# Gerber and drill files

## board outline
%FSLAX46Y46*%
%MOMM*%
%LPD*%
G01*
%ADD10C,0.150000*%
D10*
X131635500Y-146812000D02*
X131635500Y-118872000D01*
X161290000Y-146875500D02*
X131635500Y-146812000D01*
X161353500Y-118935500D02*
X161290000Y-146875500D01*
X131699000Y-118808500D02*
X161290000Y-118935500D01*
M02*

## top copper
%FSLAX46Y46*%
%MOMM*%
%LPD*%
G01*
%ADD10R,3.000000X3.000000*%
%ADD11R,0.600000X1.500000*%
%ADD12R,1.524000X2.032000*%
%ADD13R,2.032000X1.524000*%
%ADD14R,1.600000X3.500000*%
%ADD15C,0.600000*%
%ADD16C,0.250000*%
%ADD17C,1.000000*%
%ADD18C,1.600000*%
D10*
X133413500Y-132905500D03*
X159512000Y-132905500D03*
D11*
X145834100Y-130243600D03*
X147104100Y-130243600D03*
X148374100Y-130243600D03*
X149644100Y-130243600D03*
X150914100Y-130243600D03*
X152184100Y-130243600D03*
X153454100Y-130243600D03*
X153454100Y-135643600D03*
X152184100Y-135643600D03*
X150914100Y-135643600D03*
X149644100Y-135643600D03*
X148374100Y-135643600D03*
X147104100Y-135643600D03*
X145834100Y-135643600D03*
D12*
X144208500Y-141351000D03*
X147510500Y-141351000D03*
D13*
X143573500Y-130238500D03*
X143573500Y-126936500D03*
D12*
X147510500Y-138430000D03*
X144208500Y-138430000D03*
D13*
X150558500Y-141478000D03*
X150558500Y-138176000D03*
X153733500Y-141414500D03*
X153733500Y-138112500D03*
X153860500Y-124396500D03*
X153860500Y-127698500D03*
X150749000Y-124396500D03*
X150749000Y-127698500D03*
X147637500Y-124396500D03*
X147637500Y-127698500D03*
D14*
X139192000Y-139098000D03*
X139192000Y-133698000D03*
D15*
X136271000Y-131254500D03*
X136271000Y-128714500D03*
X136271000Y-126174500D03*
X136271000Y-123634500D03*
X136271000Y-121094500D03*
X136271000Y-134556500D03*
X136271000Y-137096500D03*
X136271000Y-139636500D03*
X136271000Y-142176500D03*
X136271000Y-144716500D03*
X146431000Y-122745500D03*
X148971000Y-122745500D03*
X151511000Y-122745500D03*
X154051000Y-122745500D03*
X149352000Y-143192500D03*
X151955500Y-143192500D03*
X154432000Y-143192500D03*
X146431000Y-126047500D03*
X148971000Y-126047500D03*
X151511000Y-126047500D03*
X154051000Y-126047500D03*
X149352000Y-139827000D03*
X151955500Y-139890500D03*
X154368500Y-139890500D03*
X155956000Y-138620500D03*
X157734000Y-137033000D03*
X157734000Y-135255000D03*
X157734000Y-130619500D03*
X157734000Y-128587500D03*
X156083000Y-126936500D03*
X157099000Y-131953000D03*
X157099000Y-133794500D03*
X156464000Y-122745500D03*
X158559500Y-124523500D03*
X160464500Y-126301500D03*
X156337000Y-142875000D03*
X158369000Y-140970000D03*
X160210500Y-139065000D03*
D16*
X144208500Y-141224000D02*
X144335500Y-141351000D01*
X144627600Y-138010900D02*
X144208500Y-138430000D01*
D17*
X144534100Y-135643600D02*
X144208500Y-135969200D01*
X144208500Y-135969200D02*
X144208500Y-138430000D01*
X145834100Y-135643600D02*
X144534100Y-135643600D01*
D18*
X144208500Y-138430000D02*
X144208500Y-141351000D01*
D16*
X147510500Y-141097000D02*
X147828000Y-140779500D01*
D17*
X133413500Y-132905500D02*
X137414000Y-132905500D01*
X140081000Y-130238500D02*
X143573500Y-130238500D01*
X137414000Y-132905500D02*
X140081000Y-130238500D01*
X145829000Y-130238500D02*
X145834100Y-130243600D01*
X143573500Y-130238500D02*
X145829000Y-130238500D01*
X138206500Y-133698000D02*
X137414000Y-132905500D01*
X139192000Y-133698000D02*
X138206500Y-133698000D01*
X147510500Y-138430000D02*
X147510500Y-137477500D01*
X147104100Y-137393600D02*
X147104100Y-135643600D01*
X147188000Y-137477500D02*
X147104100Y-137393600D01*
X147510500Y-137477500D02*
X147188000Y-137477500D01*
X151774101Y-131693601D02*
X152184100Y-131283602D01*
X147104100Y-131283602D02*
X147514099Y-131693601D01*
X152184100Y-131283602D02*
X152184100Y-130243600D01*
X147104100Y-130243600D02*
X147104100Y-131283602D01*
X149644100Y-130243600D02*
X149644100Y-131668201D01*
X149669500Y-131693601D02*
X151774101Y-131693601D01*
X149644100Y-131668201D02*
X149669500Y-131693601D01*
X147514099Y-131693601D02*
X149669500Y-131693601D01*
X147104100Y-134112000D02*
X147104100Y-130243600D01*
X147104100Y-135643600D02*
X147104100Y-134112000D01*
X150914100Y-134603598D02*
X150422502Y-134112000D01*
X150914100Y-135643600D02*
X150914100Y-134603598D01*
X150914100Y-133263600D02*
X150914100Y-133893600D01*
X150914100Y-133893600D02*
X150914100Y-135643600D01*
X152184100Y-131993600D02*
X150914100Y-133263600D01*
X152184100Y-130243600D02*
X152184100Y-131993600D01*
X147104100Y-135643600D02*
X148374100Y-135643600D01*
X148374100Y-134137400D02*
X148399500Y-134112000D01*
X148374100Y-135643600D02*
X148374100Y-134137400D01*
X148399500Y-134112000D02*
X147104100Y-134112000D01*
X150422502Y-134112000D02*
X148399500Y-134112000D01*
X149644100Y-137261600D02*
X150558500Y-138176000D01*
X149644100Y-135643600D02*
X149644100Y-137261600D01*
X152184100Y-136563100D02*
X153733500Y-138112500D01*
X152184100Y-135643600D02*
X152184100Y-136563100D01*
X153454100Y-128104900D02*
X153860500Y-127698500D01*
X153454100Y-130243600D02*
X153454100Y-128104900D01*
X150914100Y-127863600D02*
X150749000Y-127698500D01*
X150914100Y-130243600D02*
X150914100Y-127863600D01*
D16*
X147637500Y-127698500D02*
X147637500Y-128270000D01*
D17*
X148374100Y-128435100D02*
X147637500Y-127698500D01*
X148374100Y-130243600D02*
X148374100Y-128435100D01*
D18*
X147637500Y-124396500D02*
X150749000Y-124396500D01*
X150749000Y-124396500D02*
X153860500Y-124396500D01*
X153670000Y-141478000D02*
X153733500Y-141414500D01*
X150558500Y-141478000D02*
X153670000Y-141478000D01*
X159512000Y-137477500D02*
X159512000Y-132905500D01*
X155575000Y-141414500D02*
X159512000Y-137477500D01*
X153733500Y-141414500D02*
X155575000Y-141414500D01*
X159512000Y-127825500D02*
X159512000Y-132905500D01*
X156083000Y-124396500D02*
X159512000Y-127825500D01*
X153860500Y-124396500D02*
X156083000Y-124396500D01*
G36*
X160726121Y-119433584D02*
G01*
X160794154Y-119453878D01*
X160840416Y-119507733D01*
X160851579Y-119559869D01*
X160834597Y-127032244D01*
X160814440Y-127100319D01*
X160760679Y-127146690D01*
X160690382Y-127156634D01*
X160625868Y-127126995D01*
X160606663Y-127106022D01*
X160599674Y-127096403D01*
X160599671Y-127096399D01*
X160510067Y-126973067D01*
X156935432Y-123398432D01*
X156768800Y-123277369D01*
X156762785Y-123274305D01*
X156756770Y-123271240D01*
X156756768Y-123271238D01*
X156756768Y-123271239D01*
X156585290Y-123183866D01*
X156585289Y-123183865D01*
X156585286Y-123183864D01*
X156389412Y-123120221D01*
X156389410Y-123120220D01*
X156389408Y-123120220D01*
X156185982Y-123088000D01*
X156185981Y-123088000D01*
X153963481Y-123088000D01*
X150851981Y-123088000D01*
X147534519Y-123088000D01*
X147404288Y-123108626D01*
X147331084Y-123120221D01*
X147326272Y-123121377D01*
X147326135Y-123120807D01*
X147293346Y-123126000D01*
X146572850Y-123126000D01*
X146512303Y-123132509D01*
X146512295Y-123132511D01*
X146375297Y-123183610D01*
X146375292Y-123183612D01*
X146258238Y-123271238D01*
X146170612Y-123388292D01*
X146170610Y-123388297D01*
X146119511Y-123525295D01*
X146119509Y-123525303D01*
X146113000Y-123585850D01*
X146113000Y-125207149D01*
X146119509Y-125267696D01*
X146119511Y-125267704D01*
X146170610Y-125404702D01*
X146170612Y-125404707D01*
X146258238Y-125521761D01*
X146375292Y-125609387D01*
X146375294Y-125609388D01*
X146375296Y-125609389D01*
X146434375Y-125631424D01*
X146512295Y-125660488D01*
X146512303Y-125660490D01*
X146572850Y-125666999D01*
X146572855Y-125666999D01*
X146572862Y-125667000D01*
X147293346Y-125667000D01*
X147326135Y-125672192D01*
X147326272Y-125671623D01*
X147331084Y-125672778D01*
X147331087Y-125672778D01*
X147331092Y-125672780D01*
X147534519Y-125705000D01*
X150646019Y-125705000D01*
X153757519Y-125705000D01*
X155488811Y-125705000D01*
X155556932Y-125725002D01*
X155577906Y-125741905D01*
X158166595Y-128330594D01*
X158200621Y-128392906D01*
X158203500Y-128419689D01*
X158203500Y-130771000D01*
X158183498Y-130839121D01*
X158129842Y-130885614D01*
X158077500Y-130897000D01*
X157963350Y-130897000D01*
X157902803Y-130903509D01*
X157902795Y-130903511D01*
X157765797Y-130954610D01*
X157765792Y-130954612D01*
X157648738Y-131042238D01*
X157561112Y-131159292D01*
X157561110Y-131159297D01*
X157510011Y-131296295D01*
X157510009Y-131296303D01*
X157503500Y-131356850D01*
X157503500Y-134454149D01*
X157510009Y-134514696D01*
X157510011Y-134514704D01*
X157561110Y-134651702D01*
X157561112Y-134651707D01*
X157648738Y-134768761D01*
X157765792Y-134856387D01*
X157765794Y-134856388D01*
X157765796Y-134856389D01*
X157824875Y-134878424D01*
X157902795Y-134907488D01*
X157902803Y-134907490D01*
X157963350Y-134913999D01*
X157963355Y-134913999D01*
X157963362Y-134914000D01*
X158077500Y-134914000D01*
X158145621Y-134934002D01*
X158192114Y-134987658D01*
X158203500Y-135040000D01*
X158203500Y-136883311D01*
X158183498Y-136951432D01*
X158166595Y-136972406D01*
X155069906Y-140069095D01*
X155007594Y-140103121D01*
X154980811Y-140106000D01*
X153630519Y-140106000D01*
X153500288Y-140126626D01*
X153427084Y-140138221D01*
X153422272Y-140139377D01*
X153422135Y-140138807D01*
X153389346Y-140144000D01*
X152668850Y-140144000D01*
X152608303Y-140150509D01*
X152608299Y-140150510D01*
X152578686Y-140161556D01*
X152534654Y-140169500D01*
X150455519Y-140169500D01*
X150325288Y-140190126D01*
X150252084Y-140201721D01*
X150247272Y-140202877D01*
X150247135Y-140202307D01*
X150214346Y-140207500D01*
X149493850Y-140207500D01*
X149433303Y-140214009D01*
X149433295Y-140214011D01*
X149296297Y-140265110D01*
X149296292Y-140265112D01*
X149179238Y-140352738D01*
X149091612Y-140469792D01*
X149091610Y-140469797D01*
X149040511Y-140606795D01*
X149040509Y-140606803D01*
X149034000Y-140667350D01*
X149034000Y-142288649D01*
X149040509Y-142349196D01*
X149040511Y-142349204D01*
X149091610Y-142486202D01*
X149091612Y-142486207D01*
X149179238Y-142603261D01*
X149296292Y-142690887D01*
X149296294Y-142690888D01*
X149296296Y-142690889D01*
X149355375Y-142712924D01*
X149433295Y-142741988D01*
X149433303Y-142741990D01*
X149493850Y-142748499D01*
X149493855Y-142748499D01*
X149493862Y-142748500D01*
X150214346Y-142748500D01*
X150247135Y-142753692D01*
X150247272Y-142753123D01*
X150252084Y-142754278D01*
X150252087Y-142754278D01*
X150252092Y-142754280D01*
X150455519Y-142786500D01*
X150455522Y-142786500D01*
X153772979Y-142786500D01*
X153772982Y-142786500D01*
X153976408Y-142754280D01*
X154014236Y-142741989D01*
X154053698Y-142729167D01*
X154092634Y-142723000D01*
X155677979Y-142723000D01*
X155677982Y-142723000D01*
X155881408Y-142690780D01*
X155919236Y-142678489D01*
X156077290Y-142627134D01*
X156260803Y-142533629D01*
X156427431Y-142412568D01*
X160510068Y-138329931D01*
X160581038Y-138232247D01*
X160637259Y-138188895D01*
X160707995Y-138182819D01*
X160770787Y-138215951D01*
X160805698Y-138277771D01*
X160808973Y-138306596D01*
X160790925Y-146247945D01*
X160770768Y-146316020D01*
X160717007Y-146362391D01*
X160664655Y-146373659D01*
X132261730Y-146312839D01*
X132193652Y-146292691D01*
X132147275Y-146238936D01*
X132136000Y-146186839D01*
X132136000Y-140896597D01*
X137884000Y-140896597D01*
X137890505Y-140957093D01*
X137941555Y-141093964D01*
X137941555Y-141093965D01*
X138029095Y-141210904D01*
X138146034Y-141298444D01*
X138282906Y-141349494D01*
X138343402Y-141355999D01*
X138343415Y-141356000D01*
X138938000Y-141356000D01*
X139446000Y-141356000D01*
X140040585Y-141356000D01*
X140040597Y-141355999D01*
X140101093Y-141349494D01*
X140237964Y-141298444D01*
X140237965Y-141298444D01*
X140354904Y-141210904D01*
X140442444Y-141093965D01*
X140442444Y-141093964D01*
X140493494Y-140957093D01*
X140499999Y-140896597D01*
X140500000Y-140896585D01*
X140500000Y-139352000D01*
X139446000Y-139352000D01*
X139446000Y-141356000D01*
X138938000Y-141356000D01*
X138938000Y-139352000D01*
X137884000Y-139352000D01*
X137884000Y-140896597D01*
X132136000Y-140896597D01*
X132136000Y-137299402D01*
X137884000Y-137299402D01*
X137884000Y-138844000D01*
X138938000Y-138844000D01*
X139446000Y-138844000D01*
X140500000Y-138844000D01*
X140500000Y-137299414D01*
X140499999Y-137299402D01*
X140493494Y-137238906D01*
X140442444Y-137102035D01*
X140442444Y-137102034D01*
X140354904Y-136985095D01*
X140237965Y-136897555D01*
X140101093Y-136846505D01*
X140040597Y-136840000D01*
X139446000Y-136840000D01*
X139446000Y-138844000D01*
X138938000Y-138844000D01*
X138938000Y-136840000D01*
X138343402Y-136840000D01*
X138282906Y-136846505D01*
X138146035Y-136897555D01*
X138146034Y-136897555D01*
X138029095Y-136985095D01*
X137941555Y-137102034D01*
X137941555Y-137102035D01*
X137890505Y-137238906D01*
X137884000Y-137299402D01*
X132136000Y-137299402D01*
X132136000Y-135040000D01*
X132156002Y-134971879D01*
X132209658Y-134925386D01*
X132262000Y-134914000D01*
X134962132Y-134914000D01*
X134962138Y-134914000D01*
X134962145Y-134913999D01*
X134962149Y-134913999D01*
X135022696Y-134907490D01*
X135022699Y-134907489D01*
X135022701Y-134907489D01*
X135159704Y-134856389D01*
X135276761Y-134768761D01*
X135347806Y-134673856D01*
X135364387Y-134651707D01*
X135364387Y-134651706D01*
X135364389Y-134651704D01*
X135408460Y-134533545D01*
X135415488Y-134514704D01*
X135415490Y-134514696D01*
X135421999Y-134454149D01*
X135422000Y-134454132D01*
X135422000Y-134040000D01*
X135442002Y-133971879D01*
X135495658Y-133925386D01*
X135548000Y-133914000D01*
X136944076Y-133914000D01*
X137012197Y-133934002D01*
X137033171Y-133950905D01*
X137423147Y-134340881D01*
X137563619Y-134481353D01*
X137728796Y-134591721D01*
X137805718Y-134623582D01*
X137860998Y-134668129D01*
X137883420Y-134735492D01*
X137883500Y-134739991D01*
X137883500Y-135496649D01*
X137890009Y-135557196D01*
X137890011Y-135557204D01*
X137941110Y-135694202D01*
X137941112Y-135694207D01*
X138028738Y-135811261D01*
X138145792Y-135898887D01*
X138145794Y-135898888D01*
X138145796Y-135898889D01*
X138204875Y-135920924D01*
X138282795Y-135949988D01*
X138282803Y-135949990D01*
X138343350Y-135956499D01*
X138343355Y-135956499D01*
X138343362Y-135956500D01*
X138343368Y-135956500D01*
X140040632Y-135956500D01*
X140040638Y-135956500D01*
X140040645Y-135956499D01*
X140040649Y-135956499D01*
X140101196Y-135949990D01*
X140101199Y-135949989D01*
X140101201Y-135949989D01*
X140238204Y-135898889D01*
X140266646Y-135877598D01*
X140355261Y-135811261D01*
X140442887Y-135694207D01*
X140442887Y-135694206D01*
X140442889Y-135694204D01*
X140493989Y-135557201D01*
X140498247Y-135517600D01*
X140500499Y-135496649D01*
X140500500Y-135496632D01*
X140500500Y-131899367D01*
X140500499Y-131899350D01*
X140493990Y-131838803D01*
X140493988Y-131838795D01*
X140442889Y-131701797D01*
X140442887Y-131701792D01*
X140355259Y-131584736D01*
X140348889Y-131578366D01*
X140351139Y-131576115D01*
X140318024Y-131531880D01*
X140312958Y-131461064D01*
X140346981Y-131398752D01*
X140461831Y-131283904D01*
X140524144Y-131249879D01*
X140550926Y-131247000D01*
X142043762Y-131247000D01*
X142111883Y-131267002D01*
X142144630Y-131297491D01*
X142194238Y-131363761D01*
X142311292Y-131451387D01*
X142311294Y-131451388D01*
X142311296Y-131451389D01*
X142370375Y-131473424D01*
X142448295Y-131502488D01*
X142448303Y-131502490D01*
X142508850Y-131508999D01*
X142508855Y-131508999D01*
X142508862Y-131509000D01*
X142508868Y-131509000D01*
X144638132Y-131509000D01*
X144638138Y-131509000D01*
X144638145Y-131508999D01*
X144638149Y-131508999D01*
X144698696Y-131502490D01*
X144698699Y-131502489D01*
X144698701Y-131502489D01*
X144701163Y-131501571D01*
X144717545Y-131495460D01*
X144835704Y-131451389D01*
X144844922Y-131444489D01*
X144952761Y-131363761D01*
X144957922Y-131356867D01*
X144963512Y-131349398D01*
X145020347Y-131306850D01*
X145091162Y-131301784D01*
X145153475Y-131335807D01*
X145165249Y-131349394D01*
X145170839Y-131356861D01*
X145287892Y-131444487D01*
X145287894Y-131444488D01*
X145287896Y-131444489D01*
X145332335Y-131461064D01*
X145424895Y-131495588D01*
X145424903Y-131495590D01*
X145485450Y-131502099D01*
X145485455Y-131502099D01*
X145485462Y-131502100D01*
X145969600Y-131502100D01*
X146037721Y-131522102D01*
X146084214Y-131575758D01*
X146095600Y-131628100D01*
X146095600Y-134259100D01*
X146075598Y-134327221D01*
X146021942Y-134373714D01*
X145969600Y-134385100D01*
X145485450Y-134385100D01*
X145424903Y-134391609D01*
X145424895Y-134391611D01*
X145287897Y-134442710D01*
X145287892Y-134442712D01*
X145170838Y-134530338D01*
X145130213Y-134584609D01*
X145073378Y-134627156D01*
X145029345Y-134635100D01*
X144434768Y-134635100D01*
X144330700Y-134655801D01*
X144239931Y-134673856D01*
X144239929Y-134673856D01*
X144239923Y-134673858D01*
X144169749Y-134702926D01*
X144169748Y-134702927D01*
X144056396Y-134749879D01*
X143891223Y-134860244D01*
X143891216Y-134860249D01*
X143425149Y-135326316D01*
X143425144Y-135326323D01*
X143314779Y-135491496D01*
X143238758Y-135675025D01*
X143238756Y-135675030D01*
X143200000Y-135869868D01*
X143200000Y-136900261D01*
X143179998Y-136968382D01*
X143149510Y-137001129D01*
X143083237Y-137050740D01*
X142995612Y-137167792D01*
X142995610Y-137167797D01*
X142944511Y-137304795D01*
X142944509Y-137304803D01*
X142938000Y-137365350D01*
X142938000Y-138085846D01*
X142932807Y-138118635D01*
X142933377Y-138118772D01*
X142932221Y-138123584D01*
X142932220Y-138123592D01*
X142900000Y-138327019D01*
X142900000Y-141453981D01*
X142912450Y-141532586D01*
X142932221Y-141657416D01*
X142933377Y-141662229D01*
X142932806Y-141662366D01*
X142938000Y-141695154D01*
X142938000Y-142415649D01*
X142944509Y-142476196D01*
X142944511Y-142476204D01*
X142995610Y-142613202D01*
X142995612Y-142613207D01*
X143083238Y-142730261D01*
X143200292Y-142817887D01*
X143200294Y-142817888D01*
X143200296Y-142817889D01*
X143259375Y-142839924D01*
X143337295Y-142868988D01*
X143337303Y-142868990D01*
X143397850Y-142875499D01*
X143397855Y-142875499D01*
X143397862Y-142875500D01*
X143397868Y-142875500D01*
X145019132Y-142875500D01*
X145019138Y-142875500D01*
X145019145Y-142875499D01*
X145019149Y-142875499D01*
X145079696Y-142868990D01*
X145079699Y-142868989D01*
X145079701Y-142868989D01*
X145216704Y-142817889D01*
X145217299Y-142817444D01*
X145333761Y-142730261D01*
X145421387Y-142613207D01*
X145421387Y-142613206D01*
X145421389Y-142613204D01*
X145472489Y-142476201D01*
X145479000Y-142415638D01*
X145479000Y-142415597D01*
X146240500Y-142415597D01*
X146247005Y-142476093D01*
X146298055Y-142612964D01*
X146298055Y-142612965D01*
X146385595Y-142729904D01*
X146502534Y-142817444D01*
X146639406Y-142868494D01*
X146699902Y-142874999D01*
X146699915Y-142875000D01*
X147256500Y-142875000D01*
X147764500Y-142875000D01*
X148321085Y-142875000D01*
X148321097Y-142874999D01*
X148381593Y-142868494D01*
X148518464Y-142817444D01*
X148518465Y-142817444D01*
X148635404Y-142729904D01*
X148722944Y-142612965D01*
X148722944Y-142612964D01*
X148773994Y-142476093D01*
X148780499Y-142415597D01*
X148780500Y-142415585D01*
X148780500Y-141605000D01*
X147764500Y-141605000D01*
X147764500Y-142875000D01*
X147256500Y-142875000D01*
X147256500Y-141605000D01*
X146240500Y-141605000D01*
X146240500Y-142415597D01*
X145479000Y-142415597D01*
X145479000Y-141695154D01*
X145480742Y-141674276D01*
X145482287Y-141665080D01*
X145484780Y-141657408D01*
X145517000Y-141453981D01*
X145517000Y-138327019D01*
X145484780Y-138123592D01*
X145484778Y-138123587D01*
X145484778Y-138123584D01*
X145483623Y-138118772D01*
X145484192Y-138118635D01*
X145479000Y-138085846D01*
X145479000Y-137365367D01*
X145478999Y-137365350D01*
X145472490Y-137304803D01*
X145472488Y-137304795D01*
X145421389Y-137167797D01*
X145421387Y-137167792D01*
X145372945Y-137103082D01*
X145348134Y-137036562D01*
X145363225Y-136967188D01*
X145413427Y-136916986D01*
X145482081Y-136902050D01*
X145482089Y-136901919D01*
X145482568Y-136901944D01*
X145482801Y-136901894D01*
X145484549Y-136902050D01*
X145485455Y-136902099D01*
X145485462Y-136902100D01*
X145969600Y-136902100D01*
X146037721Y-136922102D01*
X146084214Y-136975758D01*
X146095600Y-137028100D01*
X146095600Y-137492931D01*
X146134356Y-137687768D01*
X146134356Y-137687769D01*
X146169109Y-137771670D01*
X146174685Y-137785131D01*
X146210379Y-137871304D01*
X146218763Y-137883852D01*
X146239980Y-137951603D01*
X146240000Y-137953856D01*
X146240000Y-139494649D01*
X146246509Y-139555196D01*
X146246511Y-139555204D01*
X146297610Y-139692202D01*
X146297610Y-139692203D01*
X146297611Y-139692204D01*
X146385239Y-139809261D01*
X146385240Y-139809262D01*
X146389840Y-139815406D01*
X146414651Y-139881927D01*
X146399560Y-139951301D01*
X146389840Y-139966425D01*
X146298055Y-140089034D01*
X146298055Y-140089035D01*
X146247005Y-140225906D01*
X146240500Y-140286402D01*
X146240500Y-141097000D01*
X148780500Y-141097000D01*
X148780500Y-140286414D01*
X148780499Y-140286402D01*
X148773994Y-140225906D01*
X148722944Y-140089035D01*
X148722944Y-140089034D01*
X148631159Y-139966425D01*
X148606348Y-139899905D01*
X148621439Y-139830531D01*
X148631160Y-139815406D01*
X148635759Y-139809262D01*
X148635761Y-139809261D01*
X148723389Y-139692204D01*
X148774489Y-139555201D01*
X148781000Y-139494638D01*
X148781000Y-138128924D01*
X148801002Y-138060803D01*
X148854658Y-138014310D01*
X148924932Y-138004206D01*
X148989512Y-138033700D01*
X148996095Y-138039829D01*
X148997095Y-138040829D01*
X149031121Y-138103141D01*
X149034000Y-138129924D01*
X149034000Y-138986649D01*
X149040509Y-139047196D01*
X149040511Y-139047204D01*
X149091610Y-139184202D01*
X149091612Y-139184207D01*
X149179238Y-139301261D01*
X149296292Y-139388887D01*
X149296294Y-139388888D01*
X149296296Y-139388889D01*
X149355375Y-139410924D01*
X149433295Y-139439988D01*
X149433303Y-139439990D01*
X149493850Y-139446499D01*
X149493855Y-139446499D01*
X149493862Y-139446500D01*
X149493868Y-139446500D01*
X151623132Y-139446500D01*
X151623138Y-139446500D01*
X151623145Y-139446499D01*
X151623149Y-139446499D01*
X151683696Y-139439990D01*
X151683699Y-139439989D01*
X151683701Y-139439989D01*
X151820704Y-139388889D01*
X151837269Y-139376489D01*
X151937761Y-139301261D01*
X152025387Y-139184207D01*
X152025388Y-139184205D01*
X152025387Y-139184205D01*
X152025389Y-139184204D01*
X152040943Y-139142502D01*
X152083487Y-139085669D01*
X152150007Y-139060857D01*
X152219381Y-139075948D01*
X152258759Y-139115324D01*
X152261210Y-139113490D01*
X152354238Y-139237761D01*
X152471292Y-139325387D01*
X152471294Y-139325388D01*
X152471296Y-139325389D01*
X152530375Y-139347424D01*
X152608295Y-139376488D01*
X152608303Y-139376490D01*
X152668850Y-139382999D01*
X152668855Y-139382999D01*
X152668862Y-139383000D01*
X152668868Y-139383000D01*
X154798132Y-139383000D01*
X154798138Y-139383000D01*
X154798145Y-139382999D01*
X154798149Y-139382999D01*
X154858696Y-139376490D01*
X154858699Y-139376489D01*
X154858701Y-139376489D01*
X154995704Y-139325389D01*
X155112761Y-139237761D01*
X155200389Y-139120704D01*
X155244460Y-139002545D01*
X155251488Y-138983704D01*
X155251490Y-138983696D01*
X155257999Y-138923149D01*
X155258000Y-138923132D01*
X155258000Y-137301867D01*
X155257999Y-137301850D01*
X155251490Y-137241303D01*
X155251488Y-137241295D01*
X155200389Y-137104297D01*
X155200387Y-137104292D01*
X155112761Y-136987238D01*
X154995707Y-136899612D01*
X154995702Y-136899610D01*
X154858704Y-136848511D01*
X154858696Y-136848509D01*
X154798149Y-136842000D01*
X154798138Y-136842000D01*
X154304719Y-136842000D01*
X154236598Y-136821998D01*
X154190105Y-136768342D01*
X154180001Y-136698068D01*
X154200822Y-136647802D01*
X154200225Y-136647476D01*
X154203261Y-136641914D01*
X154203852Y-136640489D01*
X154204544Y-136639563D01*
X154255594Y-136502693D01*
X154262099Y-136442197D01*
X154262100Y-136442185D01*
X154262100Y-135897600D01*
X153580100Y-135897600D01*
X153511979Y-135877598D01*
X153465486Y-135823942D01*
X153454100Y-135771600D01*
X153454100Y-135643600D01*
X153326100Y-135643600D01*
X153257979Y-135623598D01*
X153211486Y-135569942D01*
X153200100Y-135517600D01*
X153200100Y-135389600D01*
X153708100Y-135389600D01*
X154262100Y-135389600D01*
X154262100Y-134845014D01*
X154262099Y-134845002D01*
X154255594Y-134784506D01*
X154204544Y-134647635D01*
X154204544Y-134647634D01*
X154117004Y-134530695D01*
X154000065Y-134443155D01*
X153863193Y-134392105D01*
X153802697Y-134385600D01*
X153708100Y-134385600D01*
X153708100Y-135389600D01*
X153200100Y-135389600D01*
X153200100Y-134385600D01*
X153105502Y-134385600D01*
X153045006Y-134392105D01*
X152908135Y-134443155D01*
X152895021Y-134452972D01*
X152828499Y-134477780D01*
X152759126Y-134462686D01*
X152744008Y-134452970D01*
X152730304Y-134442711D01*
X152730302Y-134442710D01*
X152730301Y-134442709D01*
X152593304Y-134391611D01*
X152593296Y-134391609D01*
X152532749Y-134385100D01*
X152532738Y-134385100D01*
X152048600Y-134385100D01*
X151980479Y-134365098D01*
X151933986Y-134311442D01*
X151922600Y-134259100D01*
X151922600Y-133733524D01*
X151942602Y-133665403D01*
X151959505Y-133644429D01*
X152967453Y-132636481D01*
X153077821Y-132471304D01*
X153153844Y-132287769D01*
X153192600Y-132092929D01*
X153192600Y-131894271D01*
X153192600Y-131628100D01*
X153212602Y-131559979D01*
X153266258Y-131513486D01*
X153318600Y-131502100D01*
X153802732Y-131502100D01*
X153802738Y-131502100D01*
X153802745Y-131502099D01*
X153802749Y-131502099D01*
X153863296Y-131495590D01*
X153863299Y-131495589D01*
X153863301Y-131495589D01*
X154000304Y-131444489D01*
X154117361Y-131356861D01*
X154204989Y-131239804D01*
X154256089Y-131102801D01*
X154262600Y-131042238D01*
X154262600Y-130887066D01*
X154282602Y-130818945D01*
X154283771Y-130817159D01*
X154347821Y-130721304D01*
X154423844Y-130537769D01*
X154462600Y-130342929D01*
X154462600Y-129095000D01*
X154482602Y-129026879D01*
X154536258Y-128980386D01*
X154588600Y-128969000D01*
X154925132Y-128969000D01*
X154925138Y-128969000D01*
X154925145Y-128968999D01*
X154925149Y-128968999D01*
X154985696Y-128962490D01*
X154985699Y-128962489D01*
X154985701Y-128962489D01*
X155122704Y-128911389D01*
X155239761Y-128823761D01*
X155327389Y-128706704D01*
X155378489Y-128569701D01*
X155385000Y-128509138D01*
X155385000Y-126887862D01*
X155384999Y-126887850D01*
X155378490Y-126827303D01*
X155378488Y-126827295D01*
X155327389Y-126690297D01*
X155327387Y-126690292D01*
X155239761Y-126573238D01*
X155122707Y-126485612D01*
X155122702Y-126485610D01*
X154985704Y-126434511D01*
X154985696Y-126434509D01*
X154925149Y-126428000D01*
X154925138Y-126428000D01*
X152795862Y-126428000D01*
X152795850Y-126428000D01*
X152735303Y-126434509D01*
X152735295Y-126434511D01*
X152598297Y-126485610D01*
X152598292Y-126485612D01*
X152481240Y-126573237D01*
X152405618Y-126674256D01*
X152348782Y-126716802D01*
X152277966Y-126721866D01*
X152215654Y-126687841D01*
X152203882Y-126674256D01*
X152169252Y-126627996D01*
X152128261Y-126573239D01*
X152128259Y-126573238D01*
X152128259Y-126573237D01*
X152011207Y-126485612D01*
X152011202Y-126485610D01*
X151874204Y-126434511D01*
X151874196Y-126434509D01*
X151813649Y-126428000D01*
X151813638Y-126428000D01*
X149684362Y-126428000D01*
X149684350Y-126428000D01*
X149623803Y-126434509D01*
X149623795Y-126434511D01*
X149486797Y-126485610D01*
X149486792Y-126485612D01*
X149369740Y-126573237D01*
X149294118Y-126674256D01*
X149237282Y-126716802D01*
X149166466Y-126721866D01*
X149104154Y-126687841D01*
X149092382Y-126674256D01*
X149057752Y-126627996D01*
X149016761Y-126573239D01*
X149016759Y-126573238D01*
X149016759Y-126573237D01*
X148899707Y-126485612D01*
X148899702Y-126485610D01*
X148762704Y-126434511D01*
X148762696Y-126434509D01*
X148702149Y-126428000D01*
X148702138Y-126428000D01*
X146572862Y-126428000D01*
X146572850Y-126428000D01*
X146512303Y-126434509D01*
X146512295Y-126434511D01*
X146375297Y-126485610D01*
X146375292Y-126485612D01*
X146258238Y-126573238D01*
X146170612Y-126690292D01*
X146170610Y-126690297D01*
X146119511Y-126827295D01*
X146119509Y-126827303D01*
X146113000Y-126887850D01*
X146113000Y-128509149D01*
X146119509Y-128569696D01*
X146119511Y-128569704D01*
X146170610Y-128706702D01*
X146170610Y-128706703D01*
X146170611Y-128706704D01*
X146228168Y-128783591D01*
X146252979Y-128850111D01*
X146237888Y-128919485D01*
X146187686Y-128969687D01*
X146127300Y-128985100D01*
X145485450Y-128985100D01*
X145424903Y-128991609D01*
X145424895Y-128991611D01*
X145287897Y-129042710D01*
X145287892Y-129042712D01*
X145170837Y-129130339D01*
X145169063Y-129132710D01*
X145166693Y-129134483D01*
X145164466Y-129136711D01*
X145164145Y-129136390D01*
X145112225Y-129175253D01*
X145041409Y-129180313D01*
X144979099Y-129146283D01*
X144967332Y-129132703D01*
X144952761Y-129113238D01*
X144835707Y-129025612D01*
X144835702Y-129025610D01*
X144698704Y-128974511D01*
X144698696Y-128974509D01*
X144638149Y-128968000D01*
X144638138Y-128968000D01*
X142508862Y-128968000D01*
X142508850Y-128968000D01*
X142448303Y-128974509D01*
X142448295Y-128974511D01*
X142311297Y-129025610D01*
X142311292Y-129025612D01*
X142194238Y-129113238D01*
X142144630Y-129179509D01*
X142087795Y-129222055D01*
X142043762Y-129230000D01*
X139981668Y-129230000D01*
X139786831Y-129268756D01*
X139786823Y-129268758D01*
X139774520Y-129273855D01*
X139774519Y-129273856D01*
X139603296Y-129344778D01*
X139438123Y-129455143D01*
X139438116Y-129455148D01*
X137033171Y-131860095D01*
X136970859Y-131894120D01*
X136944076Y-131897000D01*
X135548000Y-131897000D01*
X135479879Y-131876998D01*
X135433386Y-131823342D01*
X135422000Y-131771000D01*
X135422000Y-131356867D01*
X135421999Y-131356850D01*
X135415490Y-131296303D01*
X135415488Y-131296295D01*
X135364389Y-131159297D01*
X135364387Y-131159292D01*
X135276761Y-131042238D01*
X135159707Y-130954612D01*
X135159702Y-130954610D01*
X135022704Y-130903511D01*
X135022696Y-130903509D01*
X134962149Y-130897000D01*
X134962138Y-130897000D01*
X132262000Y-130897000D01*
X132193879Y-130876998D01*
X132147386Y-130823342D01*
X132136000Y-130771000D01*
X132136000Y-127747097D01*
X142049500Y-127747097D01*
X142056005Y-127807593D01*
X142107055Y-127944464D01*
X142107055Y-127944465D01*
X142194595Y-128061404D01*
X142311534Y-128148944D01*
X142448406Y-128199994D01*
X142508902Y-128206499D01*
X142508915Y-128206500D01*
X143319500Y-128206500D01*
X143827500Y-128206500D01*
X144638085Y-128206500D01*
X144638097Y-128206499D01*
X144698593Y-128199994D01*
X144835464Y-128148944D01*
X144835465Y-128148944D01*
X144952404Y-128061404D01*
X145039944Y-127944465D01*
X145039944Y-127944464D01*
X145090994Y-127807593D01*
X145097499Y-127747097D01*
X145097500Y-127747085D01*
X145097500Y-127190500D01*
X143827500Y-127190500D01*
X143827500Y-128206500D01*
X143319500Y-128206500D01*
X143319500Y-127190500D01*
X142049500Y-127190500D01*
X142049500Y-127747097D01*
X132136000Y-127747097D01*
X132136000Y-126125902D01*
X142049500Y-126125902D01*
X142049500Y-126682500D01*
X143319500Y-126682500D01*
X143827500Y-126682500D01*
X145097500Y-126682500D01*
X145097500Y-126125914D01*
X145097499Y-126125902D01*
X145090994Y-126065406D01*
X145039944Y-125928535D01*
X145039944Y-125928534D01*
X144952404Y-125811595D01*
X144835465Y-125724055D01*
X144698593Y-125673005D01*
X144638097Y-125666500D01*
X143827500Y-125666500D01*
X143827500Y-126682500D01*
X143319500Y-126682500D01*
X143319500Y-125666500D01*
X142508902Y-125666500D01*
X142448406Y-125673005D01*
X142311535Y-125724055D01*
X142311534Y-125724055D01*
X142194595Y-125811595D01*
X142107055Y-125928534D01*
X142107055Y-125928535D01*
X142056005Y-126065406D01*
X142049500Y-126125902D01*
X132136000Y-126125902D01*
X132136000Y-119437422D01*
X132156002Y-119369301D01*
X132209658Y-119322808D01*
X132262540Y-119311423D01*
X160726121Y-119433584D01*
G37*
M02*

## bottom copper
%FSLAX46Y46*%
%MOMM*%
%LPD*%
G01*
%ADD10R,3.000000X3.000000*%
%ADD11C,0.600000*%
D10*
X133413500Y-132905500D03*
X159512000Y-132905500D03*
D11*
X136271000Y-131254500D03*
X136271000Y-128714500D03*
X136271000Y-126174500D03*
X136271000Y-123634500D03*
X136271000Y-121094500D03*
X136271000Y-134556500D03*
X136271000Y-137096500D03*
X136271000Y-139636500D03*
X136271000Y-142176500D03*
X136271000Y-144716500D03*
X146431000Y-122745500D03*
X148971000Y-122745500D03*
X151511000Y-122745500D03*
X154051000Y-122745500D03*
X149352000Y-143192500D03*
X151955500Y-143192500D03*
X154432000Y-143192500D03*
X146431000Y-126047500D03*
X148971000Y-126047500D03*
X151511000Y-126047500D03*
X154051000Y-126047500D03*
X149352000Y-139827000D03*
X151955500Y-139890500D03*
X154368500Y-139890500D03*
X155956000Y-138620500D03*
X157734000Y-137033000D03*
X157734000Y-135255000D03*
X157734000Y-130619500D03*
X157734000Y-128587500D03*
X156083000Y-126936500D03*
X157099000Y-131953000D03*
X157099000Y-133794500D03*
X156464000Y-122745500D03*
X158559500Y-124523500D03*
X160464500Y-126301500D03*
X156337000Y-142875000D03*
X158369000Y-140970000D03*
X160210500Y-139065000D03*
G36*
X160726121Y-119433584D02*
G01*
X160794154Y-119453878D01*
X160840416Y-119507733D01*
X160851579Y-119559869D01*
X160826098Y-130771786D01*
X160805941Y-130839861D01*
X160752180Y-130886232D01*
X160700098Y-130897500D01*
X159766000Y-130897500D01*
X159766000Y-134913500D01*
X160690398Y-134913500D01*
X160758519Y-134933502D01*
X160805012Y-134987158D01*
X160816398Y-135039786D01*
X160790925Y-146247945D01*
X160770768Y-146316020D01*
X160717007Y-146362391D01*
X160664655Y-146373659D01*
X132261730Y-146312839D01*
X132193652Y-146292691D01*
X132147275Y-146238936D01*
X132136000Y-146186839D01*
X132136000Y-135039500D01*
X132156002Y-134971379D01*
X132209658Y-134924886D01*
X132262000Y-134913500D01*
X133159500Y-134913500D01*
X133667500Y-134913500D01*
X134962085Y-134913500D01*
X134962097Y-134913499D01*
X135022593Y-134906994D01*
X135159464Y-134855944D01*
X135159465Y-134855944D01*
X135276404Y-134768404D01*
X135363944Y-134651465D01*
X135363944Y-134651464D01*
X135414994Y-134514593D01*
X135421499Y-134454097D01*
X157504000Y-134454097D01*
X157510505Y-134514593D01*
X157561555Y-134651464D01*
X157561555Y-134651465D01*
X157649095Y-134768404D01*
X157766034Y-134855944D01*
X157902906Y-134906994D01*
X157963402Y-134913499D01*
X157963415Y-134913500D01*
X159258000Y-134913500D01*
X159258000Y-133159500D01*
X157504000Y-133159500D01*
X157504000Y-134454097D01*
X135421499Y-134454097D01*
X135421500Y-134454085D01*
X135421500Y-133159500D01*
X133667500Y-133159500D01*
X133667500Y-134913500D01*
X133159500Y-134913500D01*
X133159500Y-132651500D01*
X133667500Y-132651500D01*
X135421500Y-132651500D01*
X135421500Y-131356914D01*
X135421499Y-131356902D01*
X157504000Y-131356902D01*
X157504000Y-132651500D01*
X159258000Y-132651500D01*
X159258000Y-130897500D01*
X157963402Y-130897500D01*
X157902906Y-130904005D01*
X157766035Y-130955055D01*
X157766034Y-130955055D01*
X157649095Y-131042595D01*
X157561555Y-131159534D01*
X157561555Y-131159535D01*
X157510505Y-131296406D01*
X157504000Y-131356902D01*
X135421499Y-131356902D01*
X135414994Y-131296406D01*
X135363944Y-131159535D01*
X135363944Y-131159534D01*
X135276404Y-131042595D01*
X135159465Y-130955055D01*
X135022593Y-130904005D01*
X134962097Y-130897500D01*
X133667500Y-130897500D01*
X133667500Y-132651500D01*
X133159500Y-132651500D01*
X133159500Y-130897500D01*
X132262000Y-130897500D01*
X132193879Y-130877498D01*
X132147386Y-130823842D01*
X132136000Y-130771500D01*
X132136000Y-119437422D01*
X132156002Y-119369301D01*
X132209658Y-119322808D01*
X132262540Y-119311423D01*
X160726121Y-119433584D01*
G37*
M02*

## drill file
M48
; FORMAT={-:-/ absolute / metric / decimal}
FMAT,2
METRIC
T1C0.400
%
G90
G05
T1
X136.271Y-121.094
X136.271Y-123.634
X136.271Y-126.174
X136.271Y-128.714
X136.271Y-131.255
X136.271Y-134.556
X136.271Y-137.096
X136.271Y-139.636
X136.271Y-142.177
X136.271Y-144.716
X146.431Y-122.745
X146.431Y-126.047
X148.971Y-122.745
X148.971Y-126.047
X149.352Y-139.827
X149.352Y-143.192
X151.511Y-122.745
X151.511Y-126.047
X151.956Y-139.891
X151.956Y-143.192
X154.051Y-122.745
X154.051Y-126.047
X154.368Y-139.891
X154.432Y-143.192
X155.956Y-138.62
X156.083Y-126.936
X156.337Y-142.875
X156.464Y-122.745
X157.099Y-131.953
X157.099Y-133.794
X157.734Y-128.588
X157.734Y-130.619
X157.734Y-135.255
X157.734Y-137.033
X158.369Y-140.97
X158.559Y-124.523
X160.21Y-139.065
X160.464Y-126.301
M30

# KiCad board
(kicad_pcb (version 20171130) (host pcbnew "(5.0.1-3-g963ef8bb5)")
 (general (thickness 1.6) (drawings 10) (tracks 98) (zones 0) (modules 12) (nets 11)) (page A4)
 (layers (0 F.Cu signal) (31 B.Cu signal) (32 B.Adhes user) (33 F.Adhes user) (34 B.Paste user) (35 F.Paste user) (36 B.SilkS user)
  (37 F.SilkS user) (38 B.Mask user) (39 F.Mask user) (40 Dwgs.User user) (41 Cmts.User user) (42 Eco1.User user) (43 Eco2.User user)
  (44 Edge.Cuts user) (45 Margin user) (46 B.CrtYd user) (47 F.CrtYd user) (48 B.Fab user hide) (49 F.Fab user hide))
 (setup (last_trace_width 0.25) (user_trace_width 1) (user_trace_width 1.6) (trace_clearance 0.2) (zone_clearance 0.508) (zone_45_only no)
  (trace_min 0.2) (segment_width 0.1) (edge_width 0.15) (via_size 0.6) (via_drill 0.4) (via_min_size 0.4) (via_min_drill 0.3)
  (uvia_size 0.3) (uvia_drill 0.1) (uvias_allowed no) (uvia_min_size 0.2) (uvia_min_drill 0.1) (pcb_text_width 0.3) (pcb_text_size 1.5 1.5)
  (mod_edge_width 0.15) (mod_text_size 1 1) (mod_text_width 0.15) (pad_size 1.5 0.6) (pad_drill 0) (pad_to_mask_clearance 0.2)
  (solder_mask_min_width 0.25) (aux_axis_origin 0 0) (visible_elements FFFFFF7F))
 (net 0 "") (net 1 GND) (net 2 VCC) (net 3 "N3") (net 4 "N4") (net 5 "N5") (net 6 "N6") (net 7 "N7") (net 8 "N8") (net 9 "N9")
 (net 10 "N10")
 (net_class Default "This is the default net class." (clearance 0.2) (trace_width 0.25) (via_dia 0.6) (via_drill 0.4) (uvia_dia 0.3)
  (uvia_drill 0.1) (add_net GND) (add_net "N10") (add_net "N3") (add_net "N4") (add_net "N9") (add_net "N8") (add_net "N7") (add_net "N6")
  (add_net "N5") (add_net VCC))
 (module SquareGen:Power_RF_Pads (layer F.Cu) (at 133.4135 132.9055)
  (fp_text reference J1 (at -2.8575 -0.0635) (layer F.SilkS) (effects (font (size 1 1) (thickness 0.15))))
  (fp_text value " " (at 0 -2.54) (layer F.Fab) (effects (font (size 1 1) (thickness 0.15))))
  (pad 2 smd rect (at 0 0) (size 3 3) (layers B.Cu B.Paste B.Mask) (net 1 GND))
  (pad 1 smd rect (at 0 0) (size 3 3) (layers F.Cu F.Paste F.Mask) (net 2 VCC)))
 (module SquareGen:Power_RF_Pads (layer F.Cu) (at 159.512 132.9055)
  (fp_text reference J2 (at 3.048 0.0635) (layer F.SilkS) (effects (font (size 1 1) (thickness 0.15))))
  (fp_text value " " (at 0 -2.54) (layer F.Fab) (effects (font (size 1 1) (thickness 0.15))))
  (pad 2 smd rect (at 0 0) (size 3 3) (layers B.Cu B.Paste B.Mask) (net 1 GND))
  (pad 1 smd rect (at 0 0) (size 3 3) (layers F.Cu F.Paste F.Mask) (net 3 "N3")))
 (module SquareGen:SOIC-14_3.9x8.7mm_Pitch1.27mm (layer F.Cu) (at 149.6441 132.9436 90)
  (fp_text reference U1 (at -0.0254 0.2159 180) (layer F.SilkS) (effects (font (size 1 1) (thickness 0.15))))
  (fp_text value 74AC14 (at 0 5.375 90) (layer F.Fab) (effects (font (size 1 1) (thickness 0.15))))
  (pad 14 smd rect (at 2.7 -3.81 90) (size 1.5 0.6) (layers F.Cu F.Paste F.Mask) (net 2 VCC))
  (pad 13 smd rect (at 2.7 -2.54 90) (size 1.5 0.6) (layers F.Cu F.Paste F.Mask) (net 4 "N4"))
  (pad 12 smd rect (at 2.7 -1.27 90) (size 1.5 0.6) (layers F.Cu F.Paste F.Mask) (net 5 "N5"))
  (pad 11 smd rect (at 2.7 0 90) (size 1.5 0.6) (layers F.Cu F.Paste F.Mask) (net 4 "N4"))
  (pad 10 smd rect (at 2.7 1.27 90) (size 1.5 0.6) (layers F.Cu F.Paste F.Mask) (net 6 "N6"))
  (pad 9 smd rect (at 2.7 2.54 90) (size 1.5 0.6) (layers F.Cu F.Paste F.Mask) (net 4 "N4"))
  (pad 8 smd rect (at 2.7 3.81 90) (size 1.5 0.6) (layers F.Cu F.Paste F.Mask) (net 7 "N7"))
  (pad 7 smd rect (at -2.7 3.81 90) (size 1.5 0.6) (layers F.Cu F.Paste F.Mask) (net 1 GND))
  (pad 6 smd rect (at -2.7 2.54 90) (size 1.5 0.6) (layers F.Cu F.Paste F.Mask) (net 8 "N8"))
  (pad 5 smd rect (at -2.7 1.27 90) (size 1.5 0.6) (layers F.Cu F.Paste F.Mask) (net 4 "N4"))
  (pad 4 smd rect (at -2.7 0 90) (size 1.5 0.6) (layers F.Cu F.Paste F.Mask) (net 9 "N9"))
  (pad 3 smd rect (at -2.7 -1.27 90) (size 1.5 0.6) (layers F.Cu F.Paste F.Mask) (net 4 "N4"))
  (pad 2 smd rect (at -2.7 -2.54 90) (size 1.5 0.6) (layers F.Cu F.Paste F.Mask) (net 4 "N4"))
  (pad 1 smd rect (at -2.7 -3.81 90) (size 1.5 0.6) (layers F.Cu F.Paste F.Mask) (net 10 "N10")))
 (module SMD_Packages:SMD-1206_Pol (layer F.Cu) (at 145.8595 141.351)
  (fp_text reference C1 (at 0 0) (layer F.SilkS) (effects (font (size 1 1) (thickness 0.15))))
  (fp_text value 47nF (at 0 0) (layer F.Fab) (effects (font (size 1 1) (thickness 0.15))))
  (pad 1 smd rect (at -1.651 0) (size 1.524 2.032) (layers F.Cu F.Paste F.Mask) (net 10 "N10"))
  (pad 2 smd rect (at 1.651 0) (size 1.524 2.032) (layers F.Cu F.Paste F.Mask) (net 1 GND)))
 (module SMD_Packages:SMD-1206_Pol (layer F.Cu) (at 143.5735 128.5875 90)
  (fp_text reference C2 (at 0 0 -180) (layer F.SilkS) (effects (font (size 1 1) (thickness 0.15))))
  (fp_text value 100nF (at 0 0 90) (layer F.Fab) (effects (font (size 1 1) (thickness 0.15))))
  (pad 1 smd rect (at -1.651 0 90) (size 1.524 2.032) (layers F.Cu F.Paste F.Mask) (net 2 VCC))
  (pad 2 smd rect (at 1.651 0 90) (size 1.524 2.032) (layers F.Cu F.Paste F.Mask) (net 1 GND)))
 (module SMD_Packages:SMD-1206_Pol (layer F.Cu) (at 145.8595 138.43 180)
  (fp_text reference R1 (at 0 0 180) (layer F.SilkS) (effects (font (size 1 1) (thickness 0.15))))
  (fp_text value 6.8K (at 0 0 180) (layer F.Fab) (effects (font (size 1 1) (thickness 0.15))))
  (pad 1 smd rect (at -1.651 0 180) (size 1.524 2.032) (layers F.Cu F.Paste F.Mask) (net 4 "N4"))
  (pad 2 smd rect (at 1.651 0 180) (size 1.524 2.032) (layers F.Cu F.Paste F.Mask) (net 10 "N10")))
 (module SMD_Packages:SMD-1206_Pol (layer F.Cu) (at 150.5585 139.827 90)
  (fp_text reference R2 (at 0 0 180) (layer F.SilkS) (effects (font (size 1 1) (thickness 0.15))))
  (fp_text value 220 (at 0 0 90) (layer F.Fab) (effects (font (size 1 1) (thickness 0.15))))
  (pad 1 smd rect (at -1.651 0 90) (size 1.524 2.032) (layers F.Cu F.Paste F.Mask) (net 3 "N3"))
  (pad 2 smd rect (at 1.651 0 90) (size 1.524 2.032) (layers F.Cu F.Paste F.Mask) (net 9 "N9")))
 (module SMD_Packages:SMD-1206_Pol (layer F.Cu) (at 153.7335 139.7635 90)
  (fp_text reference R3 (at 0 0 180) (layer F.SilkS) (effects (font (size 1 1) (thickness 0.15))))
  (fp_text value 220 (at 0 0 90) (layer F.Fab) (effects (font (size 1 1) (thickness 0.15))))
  (pad 1 smd rect (at -1.651 0 90) (size 1.524 2.032) (layers F.Cu F.Paste F.Mask) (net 3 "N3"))
  (pad 2 smd rect (at 1.651 0 90) (size 1.524 2.032) (layers F.Cu F.Paste F.Mask) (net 8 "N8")))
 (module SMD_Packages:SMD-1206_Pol (layer F.Cu) (at 153.8605 126.0475 270)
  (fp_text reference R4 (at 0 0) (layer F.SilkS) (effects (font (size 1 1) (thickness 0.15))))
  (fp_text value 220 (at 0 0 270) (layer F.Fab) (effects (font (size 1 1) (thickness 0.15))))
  (pad 1 smd rect (at -1.651 0 270) (size 1.524 2.032) (layers F.Cu F.Paste F.Mask) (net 3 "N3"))
  (pad 2 smd rect (at 1.651 0 270) (size 1.524 2.032) (layers F.Cu F.Paste F.Mask) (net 7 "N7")))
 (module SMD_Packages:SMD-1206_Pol (layer F.Cu) (at 150.749 126.0475 270)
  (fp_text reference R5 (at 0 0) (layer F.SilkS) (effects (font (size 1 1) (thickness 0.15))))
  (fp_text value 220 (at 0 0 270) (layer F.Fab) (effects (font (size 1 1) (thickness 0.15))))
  (pad 1 smd rect (at -1.651 0 270) (size 1.524 2.032) (layers F.Cu F.Paste F.Mask) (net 3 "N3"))
  (pad 2 smd rect (at 1.651 0 270) (size 1.524 2.032) (layers F.Cu F.Paste F.Mask) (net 6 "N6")))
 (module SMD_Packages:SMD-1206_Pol (layer F.Cu) (at 147.6375 126.0475 270)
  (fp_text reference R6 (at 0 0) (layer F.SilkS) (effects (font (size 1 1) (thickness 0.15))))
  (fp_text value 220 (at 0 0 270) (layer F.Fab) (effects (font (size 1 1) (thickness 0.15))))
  (pad 1 smd rect (at -1.651 0 270) (size 1.524 2.032) (layers F.Cu F.Paste F.Mask) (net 3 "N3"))
  (pad 2 smd rect (at 1.651 0 270) (size 1.524 2.032) (layers F.Cu F.Paste F.Mask) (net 5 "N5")))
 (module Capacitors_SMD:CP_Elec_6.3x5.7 (layer F.Cu) (at 139.192 136.398 270)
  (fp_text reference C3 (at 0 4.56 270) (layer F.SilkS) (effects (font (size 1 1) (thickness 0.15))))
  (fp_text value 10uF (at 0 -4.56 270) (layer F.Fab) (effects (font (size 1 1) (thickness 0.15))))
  (pad 2 smd rect (at 2.7 0 90) (size 3.5 1.6) (layers F.Cu F.Paste F.Mask) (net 1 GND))
  (pad 1 smd rect (at -2.7 0 90) (size 3.5 1.6) (layers F.Cu F.Paste F.Mask) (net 2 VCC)))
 (gr_line (start 131.6355 146.812) (end 131.6355 118.872) (angle 90) (layer Edge.Cuts) (width 0.15))
 (gr_line (start 161.29 146.8755) (end 131.6355 146.812) (angle 90) (layer Edge.Cuts) (width 0.15))
 (gr_line (start 161.3535 118.9355) (end 161.29 146.8755) (angle 90) (layer Edge.Cuts) (width 0.15))
 (gr_line (start 131.699 118.8085) (end 161.29 118.9355) (angle 90) (layer Edge.Cuts) (width 0.15))
 (segment (start 144.2085 141.224) (end 144.3355 141.351) (width 0.25) (layer F.Cu) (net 10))
 (segment (start 144.6276 138.0109) (end 144.2085 138.43) (width 0.25) (layer F.Cu) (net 10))
 (segment (start 144.5341 135.6436) (end 144.2085 135.9692) (width 1) (layer F.Cu) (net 10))
 (segment (start 144.2085 135.9692) (end 144.2085 138.43) (width 1) (layer F.Cu) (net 10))
 (segment (start 145.8341 135.6436) (end 144.5341 135.6436) (width 1) (layer F.Cu) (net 10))
 (segment (start 144.2085 138.43) (end 144.2085 141.351) (width 1.6) (layer F.Cu) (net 10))
 (via (at 136.271 131.2545) (size 0.6) (drill 0.4) (layers F.Cu B.Cu) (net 1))
 (via (at 136.271 128.7145) (size 0.6) (drill 0.4) (layers F.Cu B.Cu) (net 1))
 (via (at 136.271 126.1745) (size 0.6) (drill 0.4) (layers F.Cu B.Cu) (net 1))
 (via (at 136.271 123.6345) (size 0.6) (drill 0.4) (layers F.Cu B.Cu) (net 1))
 (via (at 136.271 121.0945) (size 0.6) (drill 0.4) (layers F.Cu B.Cu) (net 1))
 (via (at 136.271 134.5565) (size 0.6) (drill 0.4) (layers F.Cu B.Cu) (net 1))
 (via (at 136.271 137.0965) (size 0.6) (drill 0.4) (layers F.Cu B.Cu) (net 1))
 (via (at 136.271 139.6365) (size 0.6) (drill 0.4) (layers F.Cu B.Cu) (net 1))
 (via (at 136.271 142.1765) (size 0.6) (drill 0.4) (layers F.Cu B.Cu) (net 1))
 (via (at 136.271 144.7165) (size 0.6) (drill 0.4) (layers F.Cu B.Cu) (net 1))
 (via (at 146.431 122.7455) (size 0.6) (drill 0.4) (layers F.Cu B.Cu) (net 1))
 (via (at 148.971 122.7455) (size 0.6) (drill 0.4) (layers F.Cu B.Cu) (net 1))
 (via (at 151.511 122.7455) (size 0.6) (drill 0.4) (layers F.Cu B.Cu) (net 1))
 (via (at 154.051 122.7455) (size 0.6) (drill 0.4) (layers F.Cu B.Cu) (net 1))
 (via (at 149.352 143.1925) (size 0.6) (drill 0.4) (layers F.Cu B.Cu) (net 1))
 (via (at 151.9555 143.1925) (size 0.6) (drill 0.4) (layers F.Cu B.Cu) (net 1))
 (via (at 154.432 143.1925) (size 0.6) (drill 0.4) (layers F.Cu B.Cu) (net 1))
 (via (at 146.431 126.0475) (size 0.6) (drill 0.4) (layers F.Cu B.Cu) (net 1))
 (via (at 148.971 126.0475) (size 0.6) (drill 0.4) (layers F.Cu B.Cu) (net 1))
 (via (at 151.511 126.0475) (size 0.6) (drill 0.4) (layers F.Cu B.Cu) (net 1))
 (via (at 154.051 126.0475) (size 0.6) (drill 0.4) (layers F.Cu B.Cu) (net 1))
 (via (at 149.352 139.827) (size 0.6) (drill 0.4) (layers F.Cu B.Cu) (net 1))
 (via (at 151.9555 139.8905) (size 0.6) (drill 0.4) (layers F.Cu B.Cu) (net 1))
 (via (at 154.3685 139.8905) (size 0.6) (drill 0.4) (layers F.Cu B.Cu) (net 1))
 (via (at 155.956 138.6205) (size 0.6) (drill 0.4) (layers F.Cu B.Cu) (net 1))
 (via (at 157.734 137.033) (size 0.6) (drill 0.4) (layers F.Cu B.Cu) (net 1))
 (via (at 157.734 135.255) (size 0.6) (drill 0.4) (layers F.Cu B.Cu) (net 1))
 (via (at 157.734 130.6195) (size 0.6) (drill 0.4) (layers F.Cu B.Cu) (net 1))
 (via (at 157.734 128.5875) (size 0.6) (drill 0.4) (layers F.Cu B.Cu) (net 1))
 (via (at 156.083 126.9365) (size 0.6) (drill 0.4) (layers F.Cu B.Cu) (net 1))
 (via (at 157.099 131.953) (size 0.6) (drill 0.4) (layers F.Cu B.Cu) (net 1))
 (via (at 157.099 133.7945) (size 0.6) (drill 0.4) (layers F.Cu B.Cu) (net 1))
 (via (at 156.464 122.7455) (size 0.6) (drill 0.4) (layers F.Cu B.Cu) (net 1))
 (via (at 158.5595 124.5235) (size 0.6) (drill 0.4) (layers F.Cu B.Cu) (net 1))
 (via (at 160.4645 126.3015) (size 0.6) (drill 0.4) (layers F.Cu B.Cu) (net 1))
 (via (at 156.337 142.875) (size 0.6) (drill 0.4) (layers F.Cu B.Cu) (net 1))
 (via (at 158.369 140.97) (size 0.6) (drill 0.4) (layers F.Cu B.Cu) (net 1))
 (via (at 160.2105 139.065) (size 0.6) (drill 0.4) (layers F.Cu B.Cu) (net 1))
 (segment (start 147.5105 141.097) (end 147.828 140.7795) (width 0.25) (layer F.Cu) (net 1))
 (segment (start 133.4135 132.9055) (end 137.414 132.9055) (width 1) (layer F.Cu) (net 2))
 (segment (start 140.081 130.2385) (end 143.5735 130.2385) (width 1) (layer F.Cu) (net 2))
 (segment (start 137.414 132.9055) (end 140.081 130.2385) (width 1) (layer F.Cu) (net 2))
 (segment (start 145.829 130.2385) (end 145.8341 130.2436) (width 1) (layer F.Cu) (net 2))
 (segment (start 143.5735 130.2385) (end 145.829 130.2385) (width 1) (layer F.Cu) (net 2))
 (segment (start 138.2065 133.698) (end 137.414 132.9055) (width 1) (layer F.Cu) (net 2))
 (segment (start 139.192 133.698) (end 138.2065 133.698) (width 1) (layer F.Cu) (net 2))
 (segment (start 147.5105 138.43) (end 147.5105 137.4775) (width 1) (layer F.Cu) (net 4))
 (segment (start 147.1041 137.3936) (end 147.1041 135.6436) (width 1) (layer F.Cu) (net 4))
 (segment (start 147.188 137.4775) (end 147.1041 137.3936) (width 1) (layer F.Cu) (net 4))
 (segment (start 147.5105 137.4775) (end 147.188 137.4775) (width 1) (layer F.Cu) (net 4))
 (segment (start 151.774101 131.693601) (end 152.1841 131.283602) (width 1) (layer F.Cu) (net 4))
 (segment (start 147.1041 131.283602) (end 147.514099 131.693601) (width 1) (layer F.Cu) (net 4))
 (segment (start 152.1841 131.283602) (end 152.1841 130.2436) (width 1) (layer F.Cu) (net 4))
 (segment (start 147.1041 130.2436) (end 147.1041 131.283602) (width 1) (layer F.Cu) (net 4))
 (segment (start 149.6441 130.2436) (end 149.6441 131.668201) (width 1) (layer F.Cu) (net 4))
 (segment (start 149.6695 131.693601) (end 151.774101 131.693601) (width 1) (layer F.Cu) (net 4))
 (segment (start 149.6441 131.668201) (end 149.6695 131.693601) (width 1) (layer F.Cu) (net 4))
 (segment (start 147.514099 131.693601) (end 149.6695 131.693601) (width 1) (layer F.Cu) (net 4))
 (segment (start 147.1041 134.112) (end 147.1041 130.2436) (width 1) (layer F.Cu) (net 4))
 (segment (start 147.1041 135.6436) (end 147.1041 134.112) (width 1) (layer F.Cu) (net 4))
 (segment (start 150.9141 134.603598) (end 150.422502 134.112) (width 1) (layer F.Cu) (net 4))
 (segment (start 150.9141 135.6436) (end 150.9141 134.603598) (width 1) (layer F.Cu) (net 4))
 (segment (start 150.9141 133.2636) (end 150.9141 133.8936) (width 1) (layer F.Cu) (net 4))
 (segment (start 150.9141 133.8936) (end 150.9141 135.6436) (width 1) (layer F.Cu) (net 4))
 (segment (start 152.1841 131.9936) (end 150.9141 133.2636) (width 1) (layer F.Cu) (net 4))
 (segment (start 152.1841 130.2436) (end 152.1841 131.9936) (width 1) (layer F.Cu) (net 4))
 (segment (start 147.1041 135.6436) (end 148.3741 135.6436) (width 1) (layer F.Cu) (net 4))
 (segment (start 148.3741 134.1374) (end 148.3995 134.112) (width 1) (layer F.Cu) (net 4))
 (segment (start 148.3741 135.6436) (end 148.3741 134.1374) (width 1) (layer F.Cu) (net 4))
 (segment (start 148.3995 134.112) (end 147.1041 134.112) (width 1) (layer F.Cu) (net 4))
 (segment (start 150.422502 134.112) (end 148.3995 134.112) (width 1) (layer F.Cu) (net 4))
 (segment (start 149.6441 137.2616) (end 150.5585 138.176) (width 1) (layer F.Cu) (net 9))
 (segment (start 149.6441 135.6436) (end 149.6441 137.2616) (width 1) (layer F.Cu) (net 9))
 (segment (start 152.1841 136.5631) (end 153.7335 138.1125) (width 1) (layer F.Cu) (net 8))
 (segment (start 152.1841 135.6436) (end 152.1841 136.5631) (width 1) (layer F.Cu) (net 8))
 (segment (start 153.4541 128.1049) (end 153.8605 127.6985) (width 1) (layer F.Cu) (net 7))
 (segment (start 153.4541 130.2436) (end 153.4541 128.1049) (width 1) (layer F.Cu) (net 7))
 (segment (start 150.9141 127.8636) (end 150.749 127.6985) (width 1) (layer F.Cu) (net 6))
 (segment (start 150.9141 130.2436) (end 150.9141 127.8636) (width 1) (layer F.Cu) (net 6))
 (segment (start 147.6375 127.6985) (end 147.6375 128.27) (width 0.25) (layer F.Cu) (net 5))
 (segment (start 148.3741 128.4351) (end 147.6375 127.6985) (width 1) (layer F.Cu) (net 5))
 (segment (start 148.3741 130.2436) (end 148.3741 128.4351) (width 1) (layer F.Cu) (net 5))
 (segment (start 147.6375 124.3965) (end 150.749 124.3965) (width 1.6) (layer F.Cu) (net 3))
 (segment (start 150.749 124.3965) (end 153.8605 124.3965) (width 1.6) (layer F.Cu) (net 3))
 (segment (start 153.67 141.478) (end 153.7335 141.4145) (width 1.6) (layer F.Cu) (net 3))
 (segment (start 150.5585 141.478) (end 153.67 141.478) (width 1.6) (layer F.Cu) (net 3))
 (segment (start 159.512 137.4775) (end 159.512 132.9055) (width 1.6) (layer F.Cu) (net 3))
 (segment (start 155.575 141.4145) (end 159.512 137.4775) (width 1.6) (layer F.Cu) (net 3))
 (segment (start 153.7335 141.4145) (end 155.575 141.4145) (width 1.6) (layer F.Cu) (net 3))
 (segment (start 159.512 127.8255) (end 159.512 132.9055) (width 1.6) (layer F.Cu) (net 3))
 (segment (start 156.083 124.3965) (end 159.512 127.8255) (width 1.6) (layer F.Cu) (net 3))
 (segment (start 153.8605 124.3965) (end 156.083 124.3965) (width 1.6) (layer F.Cu) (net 3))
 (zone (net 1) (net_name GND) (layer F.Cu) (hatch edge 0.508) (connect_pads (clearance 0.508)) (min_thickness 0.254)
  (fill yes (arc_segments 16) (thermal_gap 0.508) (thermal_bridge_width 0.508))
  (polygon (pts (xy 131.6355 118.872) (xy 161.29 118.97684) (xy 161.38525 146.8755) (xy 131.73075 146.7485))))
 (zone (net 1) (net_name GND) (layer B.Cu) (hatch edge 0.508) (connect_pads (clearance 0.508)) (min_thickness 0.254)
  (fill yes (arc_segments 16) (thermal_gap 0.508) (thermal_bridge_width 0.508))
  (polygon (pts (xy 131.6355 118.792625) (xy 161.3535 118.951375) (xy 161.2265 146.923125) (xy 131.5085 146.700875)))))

